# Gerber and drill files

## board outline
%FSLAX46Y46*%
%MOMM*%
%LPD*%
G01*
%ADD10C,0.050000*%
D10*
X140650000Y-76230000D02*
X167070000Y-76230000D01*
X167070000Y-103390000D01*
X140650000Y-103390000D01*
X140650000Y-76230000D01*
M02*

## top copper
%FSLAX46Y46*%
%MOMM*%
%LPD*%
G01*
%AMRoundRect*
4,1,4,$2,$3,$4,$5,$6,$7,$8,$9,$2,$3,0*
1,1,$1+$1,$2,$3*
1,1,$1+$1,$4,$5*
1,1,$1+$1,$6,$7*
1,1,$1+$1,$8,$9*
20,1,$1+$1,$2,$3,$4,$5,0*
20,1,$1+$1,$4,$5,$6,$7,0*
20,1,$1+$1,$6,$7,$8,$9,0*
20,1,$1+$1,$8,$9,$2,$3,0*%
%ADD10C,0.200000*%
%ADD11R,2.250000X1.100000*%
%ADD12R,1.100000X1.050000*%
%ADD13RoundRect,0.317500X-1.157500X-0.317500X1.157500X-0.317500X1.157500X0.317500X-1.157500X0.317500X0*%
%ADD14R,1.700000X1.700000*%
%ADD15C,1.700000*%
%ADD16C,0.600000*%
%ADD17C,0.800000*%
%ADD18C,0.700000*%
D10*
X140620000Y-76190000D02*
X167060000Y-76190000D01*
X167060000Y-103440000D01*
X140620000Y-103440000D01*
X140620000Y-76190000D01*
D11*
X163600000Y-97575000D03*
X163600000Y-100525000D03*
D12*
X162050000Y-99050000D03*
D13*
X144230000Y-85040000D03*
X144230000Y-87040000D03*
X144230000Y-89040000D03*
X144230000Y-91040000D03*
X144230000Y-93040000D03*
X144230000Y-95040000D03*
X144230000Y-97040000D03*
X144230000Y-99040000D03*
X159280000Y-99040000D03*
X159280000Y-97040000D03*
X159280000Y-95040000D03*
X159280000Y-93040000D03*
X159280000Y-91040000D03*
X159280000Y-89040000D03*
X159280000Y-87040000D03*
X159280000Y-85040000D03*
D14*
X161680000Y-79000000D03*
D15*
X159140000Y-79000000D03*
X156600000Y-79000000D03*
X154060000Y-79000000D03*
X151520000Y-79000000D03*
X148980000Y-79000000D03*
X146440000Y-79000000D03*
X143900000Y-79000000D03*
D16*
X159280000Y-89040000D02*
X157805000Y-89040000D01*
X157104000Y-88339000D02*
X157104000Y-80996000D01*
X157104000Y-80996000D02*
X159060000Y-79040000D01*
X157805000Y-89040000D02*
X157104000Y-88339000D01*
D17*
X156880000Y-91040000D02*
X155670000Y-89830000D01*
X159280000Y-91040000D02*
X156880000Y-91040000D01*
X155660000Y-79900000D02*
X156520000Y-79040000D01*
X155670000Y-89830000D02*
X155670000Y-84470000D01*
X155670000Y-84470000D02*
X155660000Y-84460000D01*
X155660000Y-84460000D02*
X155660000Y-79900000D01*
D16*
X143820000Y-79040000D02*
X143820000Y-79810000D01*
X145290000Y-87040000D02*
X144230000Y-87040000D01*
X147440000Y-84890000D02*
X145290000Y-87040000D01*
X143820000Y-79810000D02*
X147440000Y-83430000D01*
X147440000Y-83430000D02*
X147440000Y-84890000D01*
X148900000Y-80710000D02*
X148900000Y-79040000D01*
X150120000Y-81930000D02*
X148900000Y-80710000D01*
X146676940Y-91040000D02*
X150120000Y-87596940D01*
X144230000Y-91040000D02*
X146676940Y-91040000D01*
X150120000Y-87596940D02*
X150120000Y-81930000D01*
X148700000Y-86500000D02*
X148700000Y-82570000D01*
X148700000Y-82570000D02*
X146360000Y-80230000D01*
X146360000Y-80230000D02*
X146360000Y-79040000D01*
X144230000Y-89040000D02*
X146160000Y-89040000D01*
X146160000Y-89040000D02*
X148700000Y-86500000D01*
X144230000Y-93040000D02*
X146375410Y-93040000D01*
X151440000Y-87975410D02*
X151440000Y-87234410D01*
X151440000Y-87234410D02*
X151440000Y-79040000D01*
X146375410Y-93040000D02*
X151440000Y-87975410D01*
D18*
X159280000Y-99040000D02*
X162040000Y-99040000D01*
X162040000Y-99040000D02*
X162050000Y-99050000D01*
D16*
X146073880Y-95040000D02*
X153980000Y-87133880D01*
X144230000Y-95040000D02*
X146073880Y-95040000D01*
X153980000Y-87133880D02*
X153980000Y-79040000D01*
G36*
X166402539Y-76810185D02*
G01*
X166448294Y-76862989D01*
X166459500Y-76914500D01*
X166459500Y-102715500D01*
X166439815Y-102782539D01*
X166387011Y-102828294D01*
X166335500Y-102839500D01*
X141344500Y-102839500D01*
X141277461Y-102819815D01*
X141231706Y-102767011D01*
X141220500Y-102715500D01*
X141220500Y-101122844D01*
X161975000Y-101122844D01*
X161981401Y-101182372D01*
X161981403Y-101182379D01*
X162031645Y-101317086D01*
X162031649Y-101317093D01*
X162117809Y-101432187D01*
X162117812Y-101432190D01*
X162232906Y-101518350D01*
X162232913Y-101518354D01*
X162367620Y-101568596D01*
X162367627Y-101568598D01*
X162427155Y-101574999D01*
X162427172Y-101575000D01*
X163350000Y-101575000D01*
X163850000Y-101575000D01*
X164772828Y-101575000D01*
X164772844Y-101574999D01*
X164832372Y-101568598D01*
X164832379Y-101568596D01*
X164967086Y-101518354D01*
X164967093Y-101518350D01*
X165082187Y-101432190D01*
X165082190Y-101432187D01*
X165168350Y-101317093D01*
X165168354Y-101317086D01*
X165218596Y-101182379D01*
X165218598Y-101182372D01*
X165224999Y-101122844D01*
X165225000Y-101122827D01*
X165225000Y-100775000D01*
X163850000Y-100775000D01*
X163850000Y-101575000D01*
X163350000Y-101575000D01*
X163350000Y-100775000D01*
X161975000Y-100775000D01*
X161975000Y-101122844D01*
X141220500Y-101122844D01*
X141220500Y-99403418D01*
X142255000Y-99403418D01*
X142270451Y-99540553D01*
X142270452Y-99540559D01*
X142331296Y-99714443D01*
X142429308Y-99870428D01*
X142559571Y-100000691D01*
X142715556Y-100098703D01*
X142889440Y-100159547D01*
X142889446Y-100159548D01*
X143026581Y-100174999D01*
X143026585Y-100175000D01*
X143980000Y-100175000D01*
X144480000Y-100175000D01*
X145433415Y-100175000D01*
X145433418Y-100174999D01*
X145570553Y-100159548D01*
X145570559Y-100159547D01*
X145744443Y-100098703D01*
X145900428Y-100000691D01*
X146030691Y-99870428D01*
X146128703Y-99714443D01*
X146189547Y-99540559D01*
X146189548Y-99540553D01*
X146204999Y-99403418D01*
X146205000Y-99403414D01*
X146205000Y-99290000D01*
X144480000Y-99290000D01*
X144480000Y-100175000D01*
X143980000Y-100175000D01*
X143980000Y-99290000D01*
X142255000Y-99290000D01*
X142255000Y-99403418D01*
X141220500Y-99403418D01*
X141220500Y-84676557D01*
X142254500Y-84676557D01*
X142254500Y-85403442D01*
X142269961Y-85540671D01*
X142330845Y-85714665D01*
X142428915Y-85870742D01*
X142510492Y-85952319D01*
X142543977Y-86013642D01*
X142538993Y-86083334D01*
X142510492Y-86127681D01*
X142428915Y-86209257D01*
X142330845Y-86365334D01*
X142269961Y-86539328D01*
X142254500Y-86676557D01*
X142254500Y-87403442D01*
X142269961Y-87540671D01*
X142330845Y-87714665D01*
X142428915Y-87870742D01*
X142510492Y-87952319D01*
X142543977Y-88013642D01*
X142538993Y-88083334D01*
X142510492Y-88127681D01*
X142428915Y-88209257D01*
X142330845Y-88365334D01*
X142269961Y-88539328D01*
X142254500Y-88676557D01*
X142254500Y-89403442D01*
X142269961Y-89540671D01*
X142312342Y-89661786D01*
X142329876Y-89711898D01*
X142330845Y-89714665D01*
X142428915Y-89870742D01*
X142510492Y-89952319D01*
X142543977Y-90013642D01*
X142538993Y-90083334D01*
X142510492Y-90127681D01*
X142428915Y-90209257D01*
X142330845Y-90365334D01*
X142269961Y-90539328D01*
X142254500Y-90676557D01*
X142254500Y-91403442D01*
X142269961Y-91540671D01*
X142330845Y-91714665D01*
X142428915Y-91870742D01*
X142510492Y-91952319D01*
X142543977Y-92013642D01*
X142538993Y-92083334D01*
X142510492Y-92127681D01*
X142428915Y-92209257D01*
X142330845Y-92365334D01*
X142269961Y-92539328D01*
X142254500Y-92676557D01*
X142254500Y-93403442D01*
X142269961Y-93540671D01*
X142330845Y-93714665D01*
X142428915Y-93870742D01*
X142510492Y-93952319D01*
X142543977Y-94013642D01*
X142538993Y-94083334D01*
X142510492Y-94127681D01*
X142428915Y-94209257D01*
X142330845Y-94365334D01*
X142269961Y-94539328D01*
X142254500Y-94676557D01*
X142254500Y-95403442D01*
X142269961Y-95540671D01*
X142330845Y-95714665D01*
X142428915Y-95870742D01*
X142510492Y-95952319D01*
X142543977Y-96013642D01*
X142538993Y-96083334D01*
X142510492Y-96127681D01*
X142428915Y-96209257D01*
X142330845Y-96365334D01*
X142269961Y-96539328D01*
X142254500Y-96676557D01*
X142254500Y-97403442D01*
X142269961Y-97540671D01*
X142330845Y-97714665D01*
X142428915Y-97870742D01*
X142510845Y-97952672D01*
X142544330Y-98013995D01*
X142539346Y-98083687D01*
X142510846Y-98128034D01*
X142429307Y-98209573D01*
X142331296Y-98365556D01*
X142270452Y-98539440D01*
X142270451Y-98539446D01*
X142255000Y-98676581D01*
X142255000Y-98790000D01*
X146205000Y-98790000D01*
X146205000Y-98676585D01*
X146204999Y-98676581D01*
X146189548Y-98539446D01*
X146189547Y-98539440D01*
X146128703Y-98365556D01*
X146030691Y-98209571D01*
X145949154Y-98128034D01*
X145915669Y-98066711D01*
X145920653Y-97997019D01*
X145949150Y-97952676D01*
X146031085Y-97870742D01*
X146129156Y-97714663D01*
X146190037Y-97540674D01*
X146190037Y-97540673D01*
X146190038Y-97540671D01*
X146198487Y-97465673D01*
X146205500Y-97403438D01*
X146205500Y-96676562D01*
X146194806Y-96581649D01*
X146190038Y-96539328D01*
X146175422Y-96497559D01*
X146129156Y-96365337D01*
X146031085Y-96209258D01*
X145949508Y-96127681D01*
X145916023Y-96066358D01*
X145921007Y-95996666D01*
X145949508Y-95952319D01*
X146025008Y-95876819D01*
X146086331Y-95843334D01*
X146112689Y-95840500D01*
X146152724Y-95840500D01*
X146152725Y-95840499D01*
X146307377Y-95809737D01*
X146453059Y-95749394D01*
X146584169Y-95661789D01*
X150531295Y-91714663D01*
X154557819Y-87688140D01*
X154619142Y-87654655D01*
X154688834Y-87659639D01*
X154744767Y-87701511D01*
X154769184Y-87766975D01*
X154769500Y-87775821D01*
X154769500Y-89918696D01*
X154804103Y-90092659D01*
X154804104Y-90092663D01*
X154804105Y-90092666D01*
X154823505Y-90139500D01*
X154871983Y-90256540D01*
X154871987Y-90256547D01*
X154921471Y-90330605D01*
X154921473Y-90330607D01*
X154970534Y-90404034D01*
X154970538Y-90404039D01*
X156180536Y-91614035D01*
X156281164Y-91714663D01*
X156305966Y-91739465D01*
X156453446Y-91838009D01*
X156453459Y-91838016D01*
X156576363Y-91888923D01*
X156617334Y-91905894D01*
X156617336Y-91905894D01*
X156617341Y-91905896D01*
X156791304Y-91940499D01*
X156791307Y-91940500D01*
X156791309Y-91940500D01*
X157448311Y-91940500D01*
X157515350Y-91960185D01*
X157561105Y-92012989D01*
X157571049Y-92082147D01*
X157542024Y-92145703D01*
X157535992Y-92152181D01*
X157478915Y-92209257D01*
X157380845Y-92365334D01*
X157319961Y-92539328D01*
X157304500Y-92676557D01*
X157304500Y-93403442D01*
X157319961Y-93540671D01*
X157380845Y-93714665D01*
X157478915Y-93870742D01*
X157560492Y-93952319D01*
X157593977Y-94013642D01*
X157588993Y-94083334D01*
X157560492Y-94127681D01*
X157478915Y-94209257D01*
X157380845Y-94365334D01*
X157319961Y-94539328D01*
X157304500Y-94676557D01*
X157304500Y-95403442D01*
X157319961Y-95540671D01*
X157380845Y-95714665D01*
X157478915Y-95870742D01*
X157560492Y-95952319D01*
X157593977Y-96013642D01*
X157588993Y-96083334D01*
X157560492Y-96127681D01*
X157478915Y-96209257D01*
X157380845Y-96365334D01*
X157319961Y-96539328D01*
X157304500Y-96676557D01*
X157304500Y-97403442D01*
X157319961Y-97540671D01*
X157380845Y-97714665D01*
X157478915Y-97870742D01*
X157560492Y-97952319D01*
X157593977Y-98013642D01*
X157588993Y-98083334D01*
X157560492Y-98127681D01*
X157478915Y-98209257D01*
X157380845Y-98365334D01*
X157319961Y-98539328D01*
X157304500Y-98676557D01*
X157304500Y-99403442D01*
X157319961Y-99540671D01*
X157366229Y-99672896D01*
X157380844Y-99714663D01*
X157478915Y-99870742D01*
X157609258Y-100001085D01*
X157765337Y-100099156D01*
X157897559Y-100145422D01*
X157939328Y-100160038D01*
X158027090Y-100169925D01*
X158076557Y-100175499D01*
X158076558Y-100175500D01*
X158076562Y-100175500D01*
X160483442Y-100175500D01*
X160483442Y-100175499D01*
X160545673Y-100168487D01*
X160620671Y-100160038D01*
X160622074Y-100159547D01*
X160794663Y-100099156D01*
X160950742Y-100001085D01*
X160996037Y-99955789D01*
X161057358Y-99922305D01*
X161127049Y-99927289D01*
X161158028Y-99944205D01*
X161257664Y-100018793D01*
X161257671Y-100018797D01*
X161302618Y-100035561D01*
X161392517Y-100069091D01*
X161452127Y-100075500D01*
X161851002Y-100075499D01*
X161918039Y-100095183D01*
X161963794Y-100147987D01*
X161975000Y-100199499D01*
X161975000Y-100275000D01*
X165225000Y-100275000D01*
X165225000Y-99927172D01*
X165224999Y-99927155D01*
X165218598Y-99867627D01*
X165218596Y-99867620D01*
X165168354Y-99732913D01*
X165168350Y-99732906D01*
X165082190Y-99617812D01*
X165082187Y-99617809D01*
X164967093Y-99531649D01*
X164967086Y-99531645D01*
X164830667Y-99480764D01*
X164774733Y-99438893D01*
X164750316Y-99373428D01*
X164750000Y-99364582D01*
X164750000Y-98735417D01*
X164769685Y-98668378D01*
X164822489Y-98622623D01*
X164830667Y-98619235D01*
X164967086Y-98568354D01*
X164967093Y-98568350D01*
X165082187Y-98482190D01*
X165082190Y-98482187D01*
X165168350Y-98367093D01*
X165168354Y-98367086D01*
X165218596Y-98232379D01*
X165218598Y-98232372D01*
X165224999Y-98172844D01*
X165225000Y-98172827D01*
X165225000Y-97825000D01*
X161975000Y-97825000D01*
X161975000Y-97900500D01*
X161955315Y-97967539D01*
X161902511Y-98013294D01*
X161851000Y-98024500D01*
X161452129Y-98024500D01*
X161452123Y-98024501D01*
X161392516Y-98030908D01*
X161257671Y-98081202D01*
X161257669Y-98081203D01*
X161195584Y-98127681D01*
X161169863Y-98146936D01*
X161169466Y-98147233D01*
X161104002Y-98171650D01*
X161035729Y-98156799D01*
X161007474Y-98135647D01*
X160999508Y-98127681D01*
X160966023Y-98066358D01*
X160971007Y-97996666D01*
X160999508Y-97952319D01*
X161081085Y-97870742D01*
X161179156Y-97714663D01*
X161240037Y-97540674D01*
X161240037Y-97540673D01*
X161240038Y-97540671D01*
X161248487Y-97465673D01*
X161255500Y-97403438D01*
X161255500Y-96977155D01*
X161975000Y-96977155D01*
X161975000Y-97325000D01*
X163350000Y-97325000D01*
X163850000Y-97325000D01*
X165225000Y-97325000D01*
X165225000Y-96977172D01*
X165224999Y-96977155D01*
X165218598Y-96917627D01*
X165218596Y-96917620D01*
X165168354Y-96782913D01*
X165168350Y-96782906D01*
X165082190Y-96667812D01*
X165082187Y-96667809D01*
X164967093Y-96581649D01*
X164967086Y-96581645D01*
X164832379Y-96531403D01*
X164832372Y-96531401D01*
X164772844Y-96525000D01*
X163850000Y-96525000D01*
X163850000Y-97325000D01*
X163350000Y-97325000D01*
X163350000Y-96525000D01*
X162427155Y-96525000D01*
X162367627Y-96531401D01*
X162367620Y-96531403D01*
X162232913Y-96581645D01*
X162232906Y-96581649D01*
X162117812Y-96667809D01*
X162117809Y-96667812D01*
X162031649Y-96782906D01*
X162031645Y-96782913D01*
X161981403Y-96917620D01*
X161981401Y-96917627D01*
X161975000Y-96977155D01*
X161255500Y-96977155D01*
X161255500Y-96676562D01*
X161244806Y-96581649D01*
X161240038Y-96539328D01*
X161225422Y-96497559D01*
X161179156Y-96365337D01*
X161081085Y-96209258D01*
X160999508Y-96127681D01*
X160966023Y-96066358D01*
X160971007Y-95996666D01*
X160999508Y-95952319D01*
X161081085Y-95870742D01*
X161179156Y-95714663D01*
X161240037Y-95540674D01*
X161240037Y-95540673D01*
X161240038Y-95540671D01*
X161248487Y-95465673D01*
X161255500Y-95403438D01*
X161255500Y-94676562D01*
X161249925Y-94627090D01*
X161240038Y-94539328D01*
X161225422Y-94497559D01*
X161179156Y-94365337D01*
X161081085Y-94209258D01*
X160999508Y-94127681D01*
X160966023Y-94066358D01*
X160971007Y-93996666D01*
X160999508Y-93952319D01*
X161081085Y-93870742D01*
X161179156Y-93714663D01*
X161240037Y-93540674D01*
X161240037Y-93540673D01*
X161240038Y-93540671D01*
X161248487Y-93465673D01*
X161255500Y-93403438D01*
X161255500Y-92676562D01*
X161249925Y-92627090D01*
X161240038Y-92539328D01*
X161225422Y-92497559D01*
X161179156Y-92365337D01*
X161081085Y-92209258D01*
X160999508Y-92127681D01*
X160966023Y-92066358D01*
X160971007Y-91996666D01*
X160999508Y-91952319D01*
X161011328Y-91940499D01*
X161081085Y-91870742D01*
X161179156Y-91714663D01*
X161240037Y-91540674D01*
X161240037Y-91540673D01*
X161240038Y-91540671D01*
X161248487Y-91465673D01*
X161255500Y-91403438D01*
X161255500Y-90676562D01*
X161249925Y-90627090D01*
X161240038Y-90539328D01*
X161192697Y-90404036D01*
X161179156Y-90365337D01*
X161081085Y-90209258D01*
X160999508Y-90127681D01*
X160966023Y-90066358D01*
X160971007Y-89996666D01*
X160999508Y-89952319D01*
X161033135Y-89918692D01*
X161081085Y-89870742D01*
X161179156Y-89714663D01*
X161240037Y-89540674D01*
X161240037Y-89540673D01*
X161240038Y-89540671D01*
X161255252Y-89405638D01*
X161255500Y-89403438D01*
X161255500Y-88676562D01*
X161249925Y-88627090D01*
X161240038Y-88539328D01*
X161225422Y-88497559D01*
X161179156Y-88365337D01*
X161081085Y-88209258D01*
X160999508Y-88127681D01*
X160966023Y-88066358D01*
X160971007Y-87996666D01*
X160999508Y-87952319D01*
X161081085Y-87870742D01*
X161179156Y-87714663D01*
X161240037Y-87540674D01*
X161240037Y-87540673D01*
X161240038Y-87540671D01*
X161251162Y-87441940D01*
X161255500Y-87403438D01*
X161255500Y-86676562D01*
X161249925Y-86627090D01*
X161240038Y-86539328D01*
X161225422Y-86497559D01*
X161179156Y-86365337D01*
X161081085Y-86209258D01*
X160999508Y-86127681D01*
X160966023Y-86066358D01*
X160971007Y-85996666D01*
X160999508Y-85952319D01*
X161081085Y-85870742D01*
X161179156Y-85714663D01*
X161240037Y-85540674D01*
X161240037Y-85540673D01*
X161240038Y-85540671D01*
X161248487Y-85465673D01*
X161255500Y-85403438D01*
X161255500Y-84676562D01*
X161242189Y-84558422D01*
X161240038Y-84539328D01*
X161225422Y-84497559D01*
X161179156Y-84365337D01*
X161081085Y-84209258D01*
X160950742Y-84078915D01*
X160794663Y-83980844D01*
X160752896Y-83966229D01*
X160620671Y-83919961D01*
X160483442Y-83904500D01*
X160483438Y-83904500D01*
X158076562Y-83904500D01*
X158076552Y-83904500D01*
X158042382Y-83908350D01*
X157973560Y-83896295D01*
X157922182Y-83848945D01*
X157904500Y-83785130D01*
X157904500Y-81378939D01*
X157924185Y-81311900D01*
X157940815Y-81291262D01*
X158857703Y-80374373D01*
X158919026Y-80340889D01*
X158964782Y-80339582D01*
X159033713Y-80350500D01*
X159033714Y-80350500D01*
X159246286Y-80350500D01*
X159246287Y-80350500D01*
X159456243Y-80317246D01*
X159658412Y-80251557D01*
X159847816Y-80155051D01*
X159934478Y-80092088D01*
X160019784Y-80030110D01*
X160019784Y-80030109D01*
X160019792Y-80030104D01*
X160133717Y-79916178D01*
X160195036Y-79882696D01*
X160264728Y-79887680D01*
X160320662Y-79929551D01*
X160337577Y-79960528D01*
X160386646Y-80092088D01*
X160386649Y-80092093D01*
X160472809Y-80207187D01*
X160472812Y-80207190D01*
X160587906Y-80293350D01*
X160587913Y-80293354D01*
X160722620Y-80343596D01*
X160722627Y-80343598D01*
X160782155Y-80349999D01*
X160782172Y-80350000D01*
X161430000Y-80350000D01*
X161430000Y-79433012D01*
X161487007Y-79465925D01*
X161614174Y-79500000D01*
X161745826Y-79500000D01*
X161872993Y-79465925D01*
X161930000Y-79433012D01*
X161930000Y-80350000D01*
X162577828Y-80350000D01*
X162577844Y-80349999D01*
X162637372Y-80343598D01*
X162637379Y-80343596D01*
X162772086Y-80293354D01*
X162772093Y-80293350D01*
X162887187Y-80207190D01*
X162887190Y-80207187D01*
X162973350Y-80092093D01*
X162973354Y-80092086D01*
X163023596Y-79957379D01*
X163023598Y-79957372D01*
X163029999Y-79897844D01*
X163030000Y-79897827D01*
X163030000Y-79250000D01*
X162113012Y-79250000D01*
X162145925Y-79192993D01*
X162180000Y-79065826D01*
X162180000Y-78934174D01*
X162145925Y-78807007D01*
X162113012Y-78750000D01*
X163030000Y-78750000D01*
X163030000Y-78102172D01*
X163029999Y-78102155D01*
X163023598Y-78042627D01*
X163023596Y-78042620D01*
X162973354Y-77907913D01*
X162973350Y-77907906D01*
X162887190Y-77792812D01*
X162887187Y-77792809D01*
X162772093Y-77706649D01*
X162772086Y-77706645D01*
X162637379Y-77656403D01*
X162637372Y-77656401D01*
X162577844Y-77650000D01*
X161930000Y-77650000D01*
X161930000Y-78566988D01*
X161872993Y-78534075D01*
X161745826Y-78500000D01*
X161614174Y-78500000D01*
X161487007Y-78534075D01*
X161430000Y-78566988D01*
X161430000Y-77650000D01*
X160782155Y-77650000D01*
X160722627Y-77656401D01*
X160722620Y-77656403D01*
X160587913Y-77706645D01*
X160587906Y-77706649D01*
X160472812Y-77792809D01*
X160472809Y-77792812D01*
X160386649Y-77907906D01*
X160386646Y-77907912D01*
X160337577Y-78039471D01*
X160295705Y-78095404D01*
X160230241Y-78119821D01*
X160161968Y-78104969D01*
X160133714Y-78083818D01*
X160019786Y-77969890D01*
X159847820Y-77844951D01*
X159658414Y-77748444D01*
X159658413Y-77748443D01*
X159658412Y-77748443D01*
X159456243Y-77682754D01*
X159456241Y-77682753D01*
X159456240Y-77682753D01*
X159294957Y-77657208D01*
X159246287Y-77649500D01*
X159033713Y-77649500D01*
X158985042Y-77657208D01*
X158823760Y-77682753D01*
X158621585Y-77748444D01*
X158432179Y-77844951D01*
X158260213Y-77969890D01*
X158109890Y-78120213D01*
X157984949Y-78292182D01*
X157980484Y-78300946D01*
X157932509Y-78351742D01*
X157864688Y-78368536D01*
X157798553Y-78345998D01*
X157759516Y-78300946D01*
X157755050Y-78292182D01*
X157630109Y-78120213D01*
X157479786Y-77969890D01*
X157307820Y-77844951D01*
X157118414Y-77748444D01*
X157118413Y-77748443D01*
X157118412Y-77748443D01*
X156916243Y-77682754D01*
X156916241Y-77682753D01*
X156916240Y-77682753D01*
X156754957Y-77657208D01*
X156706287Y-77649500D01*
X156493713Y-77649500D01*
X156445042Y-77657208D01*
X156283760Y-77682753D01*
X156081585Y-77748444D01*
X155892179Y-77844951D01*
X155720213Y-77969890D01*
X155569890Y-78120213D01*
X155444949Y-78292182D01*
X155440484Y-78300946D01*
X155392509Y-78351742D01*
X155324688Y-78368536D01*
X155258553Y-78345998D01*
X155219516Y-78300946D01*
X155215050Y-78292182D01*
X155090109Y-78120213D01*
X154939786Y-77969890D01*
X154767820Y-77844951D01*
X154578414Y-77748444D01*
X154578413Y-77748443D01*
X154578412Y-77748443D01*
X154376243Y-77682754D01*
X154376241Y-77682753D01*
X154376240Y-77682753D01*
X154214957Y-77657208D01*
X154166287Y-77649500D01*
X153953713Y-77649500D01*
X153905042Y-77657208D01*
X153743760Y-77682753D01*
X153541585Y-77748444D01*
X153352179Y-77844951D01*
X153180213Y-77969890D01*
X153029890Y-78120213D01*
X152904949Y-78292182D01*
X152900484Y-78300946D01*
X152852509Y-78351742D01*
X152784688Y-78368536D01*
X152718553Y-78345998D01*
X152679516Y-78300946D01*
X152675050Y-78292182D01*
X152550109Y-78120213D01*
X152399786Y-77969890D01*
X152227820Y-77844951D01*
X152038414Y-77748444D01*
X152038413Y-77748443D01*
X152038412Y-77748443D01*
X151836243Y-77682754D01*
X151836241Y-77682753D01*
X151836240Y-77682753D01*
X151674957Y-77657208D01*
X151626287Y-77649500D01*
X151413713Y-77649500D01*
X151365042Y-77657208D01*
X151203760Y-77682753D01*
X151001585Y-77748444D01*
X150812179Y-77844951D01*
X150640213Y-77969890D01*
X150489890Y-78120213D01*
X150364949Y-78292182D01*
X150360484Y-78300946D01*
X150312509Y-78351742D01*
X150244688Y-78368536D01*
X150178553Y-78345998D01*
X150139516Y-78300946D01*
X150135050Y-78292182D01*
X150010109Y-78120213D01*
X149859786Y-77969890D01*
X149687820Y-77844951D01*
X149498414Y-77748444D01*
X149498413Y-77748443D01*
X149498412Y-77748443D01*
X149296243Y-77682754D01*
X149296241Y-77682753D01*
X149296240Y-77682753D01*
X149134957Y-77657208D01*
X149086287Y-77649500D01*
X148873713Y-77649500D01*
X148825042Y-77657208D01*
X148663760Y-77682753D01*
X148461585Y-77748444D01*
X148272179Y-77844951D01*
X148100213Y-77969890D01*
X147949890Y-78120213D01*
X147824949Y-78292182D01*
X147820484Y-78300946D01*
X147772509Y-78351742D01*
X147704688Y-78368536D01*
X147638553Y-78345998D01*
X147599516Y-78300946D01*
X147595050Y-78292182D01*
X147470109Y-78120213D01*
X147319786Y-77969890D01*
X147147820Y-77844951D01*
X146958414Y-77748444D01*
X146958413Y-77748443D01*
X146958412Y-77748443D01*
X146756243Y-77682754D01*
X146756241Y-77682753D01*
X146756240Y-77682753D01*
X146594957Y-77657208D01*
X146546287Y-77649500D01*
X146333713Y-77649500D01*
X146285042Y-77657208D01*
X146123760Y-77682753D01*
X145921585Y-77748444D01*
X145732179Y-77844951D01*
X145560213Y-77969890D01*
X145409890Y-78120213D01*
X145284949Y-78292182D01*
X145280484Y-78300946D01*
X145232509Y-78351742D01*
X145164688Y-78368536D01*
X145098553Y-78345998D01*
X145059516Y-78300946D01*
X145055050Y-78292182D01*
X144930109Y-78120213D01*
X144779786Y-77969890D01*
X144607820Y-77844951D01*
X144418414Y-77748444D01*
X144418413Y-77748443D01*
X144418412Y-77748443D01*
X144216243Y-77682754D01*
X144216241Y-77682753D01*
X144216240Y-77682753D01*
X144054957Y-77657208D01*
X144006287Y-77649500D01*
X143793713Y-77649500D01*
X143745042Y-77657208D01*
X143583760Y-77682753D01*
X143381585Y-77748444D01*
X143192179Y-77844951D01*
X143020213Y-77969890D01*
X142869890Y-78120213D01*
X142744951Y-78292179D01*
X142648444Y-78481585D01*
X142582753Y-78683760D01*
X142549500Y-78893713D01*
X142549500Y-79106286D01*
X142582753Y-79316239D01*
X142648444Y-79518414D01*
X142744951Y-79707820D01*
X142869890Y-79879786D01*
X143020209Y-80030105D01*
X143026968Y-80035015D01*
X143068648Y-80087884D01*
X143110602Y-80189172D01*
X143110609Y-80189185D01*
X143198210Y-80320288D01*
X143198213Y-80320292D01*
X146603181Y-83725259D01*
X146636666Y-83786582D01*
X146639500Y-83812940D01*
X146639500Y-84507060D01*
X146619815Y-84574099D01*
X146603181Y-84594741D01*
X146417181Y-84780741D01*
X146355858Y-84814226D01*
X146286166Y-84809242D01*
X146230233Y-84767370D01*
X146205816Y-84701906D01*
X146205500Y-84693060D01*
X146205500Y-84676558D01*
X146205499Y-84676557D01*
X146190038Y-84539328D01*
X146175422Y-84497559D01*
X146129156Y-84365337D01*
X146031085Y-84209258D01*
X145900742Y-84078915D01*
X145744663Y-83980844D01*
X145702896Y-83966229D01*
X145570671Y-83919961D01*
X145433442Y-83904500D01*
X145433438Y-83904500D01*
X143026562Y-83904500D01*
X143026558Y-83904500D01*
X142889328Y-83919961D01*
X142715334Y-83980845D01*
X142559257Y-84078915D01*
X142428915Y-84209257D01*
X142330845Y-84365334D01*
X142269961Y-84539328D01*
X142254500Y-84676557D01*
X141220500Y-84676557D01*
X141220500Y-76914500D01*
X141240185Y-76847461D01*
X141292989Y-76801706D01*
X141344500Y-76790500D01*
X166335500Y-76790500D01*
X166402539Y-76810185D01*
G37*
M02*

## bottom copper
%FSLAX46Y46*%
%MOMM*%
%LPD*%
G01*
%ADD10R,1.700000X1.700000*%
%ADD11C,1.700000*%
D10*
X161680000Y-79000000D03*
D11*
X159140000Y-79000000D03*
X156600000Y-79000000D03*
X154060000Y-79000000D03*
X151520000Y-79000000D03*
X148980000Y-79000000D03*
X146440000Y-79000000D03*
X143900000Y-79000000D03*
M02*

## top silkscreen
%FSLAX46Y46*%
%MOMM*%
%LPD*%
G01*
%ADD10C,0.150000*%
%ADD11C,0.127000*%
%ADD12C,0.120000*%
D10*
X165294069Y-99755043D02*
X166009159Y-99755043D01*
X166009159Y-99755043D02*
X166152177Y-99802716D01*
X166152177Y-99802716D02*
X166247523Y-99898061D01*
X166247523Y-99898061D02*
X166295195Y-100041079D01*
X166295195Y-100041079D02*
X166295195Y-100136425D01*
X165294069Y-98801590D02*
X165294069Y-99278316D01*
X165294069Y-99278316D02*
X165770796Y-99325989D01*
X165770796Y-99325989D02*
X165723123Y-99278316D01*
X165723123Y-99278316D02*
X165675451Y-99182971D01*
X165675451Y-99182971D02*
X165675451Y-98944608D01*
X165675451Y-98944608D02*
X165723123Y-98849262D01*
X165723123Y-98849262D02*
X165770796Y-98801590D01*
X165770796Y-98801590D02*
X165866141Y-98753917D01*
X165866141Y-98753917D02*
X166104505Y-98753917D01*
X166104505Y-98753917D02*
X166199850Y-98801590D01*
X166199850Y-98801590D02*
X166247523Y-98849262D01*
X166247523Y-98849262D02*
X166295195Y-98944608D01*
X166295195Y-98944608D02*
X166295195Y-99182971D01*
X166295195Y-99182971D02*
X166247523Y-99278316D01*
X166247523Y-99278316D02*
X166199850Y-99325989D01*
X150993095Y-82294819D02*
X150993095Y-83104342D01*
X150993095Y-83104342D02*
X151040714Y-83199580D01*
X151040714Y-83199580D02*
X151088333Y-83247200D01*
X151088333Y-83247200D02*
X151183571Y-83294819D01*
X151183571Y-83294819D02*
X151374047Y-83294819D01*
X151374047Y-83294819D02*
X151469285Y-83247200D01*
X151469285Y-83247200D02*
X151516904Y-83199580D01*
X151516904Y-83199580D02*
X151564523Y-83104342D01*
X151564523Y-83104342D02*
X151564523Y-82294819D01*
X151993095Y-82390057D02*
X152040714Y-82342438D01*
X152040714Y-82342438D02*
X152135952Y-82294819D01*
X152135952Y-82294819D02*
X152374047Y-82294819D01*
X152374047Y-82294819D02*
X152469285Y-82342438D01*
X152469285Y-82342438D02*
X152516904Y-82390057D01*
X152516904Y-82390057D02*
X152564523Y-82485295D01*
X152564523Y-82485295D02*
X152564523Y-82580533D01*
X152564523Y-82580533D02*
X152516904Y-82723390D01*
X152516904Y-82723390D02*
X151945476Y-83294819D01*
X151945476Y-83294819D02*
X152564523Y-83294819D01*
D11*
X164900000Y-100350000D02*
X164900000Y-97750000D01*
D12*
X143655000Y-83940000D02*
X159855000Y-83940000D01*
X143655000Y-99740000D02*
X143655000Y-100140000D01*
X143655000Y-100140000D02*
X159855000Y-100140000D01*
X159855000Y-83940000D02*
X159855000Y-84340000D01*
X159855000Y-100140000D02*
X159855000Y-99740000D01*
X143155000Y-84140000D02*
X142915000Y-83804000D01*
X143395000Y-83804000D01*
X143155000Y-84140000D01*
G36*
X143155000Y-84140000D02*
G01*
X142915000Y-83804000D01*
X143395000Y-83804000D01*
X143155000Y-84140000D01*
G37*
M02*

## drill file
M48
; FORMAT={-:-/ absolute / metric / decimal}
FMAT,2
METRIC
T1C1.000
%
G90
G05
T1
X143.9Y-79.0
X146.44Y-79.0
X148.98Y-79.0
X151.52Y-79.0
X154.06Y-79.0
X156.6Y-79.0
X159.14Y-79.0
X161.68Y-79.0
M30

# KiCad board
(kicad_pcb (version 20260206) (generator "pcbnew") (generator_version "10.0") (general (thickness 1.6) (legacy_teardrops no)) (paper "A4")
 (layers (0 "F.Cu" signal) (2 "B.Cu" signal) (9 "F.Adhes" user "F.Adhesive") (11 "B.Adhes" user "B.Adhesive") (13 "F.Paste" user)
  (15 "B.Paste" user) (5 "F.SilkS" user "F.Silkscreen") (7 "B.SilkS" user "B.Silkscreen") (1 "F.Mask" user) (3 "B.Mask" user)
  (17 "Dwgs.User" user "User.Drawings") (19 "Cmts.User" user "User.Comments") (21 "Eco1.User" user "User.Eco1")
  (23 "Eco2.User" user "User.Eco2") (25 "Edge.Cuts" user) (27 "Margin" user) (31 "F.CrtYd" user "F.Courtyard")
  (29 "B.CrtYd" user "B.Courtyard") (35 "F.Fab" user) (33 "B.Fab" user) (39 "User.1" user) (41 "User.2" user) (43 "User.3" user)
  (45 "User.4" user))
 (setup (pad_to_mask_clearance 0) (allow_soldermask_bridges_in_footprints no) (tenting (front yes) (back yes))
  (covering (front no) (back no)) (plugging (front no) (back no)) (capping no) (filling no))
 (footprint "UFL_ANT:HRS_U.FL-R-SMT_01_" (layer "F.Cu") (at 163.6 99.05 -90)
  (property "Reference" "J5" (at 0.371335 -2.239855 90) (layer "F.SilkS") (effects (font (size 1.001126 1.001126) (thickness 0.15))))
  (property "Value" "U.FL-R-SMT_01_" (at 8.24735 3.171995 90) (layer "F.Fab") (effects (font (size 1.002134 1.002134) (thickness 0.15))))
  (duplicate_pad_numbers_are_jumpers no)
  (fp_line (start 1.3 -1.3) (end -1.3 -1.3) (stroke (width 0.127) (type solid)) (layer "F.SilkS"))
  (pad "1" smd rect (at -1.475 0 270) (size 1.1 2.25) (layers "F.Cu" "F.Mask" "F.Paste") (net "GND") (solder_mask_margin 0.102))
  (pad "2" smd rect (at 1.475 0 270) (size 1.1 2.25) (layers "F.Cu" "F.Mask" "F.Paste") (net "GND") (solder_mask_margin 0.102))
  (pad "3" smd rect (at 0 1.55 270) (size 1.05 1.1) (layers "F.Cu" "F.Mask" "F.Paste") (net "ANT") (solder_mask_margin 0.102))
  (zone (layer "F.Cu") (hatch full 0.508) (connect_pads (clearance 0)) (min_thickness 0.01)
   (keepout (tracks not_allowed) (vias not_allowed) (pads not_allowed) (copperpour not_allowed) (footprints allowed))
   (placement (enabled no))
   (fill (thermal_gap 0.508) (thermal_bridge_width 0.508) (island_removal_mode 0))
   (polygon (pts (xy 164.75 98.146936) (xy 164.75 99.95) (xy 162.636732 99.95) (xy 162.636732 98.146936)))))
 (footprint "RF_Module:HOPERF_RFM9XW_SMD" (layer "F.Cu") (at 151.755 92.04)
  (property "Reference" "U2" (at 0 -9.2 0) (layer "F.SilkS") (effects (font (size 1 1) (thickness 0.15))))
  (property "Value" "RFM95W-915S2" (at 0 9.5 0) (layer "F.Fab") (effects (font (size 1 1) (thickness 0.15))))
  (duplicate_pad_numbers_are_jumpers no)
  (fp_line (start -8.1 -8.1) (end 8.1 -8.1) (stroke (width 0.12) (type solid)) (layer "F.SilkS"))
  (fp_line (start -8.1 7.7) (end -8.1 8.1) (stroke (width 0.12) (type solid)) (layer "F.SilkS"))
  (fp_line (start -8.1 8.1) (end 8.1 8.1) (stroke (width 0.12) (type solid)) (layer "F.SilkS"))
  (fp_line (start 8.1 -8.1) (end 8.1 -7.7) (stroke (width 0.12) (type solid)) (layer "F.SilkS"))
  (fp_line (start 8.1 8.1) (end 8.1 7.7) (stroke (width 0.12) (type solid)) (layer "F.SilkS"))
  (fp_poly
   (pts (xy -8.6 -7.9) (xy -8.84 -8.236) (xy -8.36 -8.236) (xy -8.6 -7.9)) (stroke (width 0.12) (type solid)) (fill yes) (layer "F.SilkS"))
  (pad "1" smd roundrect (at -7.525 -7) (size 2.95 1.27) (layers "F.Cu" "F.Mask" "F.Paste") (roundrect_rratio 0.25)
   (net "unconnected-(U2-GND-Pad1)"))
  (pad "2" smd roundrect (at -7.525 -5) (size 2.95 1.27) (layers "F.Cu" "F.Mask" "F.Paste") (roundrect_rratio 0.25) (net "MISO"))
  (pad "3" smd roundrect (at -7.525 -3) (size 2.95 1.27) (layers "F.Cu" "F.Mask" "F.Paste") (roundrect_rratio 0.25) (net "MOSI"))
  (pad "4" smd roundrect (at -7.525 -1) (size 2.95 1.27) (layers "F.Cu" "F.Mask" "F.Paste") (roundrect_rratio 0.25) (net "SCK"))
  (pad "5" smd roundrect (at -7.525 1) (size 2.95 1.27) (layers "F.Cu" "F.Mask" "F.Paste") (roundrect_rratio 0.25) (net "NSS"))
  (pad "6" smd roundrect (at -7.525 3) (size 2.95 1.27) (layers "F.Cu" "F.Mask" "F.Paste") (roundrect_rratio 0.25) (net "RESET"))
  (pad "7" smd roundrect (at -7.525 5) (size 2.95 1.27) (layers "F.Cu" "F.Mask" "F.Paste") (roundrect_rratio 0.25)
   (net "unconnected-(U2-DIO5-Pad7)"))
  (pad "8" smd roundrect (at -7.525 7) (size 2.95 1.27) (layers "F.Cu" "F.Mask" "F.Paste") (roundrect_rratio 0.25) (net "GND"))
  (pad "9" smd roundrect (at 7.525 7) (size 2.95 1.27) (layers "F.Cu" "F.Mask" "F.Paste") (roundrect_rratio 0.25) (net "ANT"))
  (pad "10" smd roundrect (at 7.525 5) (size 2.95 1.27) (layers "F.Cu" "F.Mask" "F.Paste") (roundrect_rratio 0.25)
   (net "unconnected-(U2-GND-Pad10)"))
  (pad "11" smd roundrect (at 7.525 3) (size 2.95 1.27) (layers "F.Cu" "F.Mask" "F.Paste") (roundrect_rratio 0.25)
   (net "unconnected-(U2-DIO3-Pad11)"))
  (pad "12" smd roundrect (at 7.525 1) (size 2.95 1.27) (layers "F.Cu" "F.Mask" "F.Paste") (roundrect_rratio 0.25)
   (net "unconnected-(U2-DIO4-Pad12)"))
  (pad "13" smd roundrect (at 7.525 -1) (size 2.95 1.27) (layers "F.Cu" "F.Mask" "F.Paste") (roundrect_rratio 0.25) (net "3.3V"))
  (pad "14" smd roundrect (at 7.525 -3) (size 2.95 1.27) (layers "F.Cu" "F.Mask" "F.Paste") (roundrect_rratio 0.25) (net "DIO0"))
  (pad "15" smd roundrect (at 7.525 -5) (size 2.95 1.27) (layers "F.Cu" "F.Mask" "F.Paste") (roundrect_rratio 0.25)
   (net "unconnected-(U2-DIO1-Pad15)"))
  (pad "16" smd roundrect (at 7.525 -7) (size 2.95 1.27) (layers "F.Cu" "F.Mask" "F.Paste") (roundrect_rratio 0.25)
   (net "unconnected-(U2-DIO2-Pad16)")))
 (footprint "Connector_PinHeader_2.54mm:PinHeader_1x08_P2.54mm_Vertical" (layer "B.Cu") (at 161.68 79 90)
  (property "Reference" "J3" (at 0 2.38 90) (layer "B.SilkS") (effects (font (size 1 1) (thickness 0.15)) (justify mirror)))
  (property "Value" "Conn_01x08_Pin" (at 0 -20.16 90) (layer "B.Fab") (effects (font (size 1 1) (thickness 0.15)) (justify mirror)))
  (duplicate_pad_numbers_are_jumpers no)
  (pad "1" thru_hole rect (at 0 0 90) (size 1.7 1.7) (drill 1) (layers "*.Cu" "*.Mask") (remove_unused_layers no) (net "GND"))
  (pad "2" thru_hole circle (at 0 -2.54 90) (size 1.7 1.7) (drill 1) (layers "*.Cu" "*.Mask") (remove_unused_layers no) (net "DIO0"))
  (pad "3" thru_hole circle (at 0 -5.08 90) (size 1.7 1.7) (drill 1) (layers "*.Cu" "*.Mask") (remove_unused_layers no) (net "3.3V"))
  (pad "4" thru_hole circle (at 0 -7.62 90) (size 1.7 1.7) (drill 1) (layers "*.Cu" "*.Mask") (remove_unused_layers no) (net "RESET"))
  (pad "5" thru_hole circle (at 0 -10.16 90) (size 1.7 1.7) (drill 1) (layers "*.Cu" "*.Mask") (remove_unused_layers no) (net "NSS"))
  (pad "6" thru_hole circle (at 0 -12.7 90) (size 1.7 1.7) (drill 1) (layers "*.Cu" "*.Mask") (remove_unused_layers no) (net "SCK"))
  (pad "7" thru_hole circle (at 0 -15.24 90) (size 1.7 1.7) (drill 1) (layers "*.Cu" "*.Mask") (remove_unused_layers no) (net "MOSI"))
  (pad "8" thru_hole circle (at 0 -17.78 90) (size 1.7 1.7) (drill 1) (layers "*.Cu" "*.Mask") (remove_unused_layers no) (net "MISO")))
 (gr_rect (start 140.62 76.19) (end 167.06 103.44) (stroke (width 0.2) (type default)) (fill no) (layer "F.Cu") (net "DIO0"))
 (gr_rect (start 140.65 76.23) (end 167.07 103.39) (stroke (width 0.05) (type default)) (fill no) (layer "Edge.Cuts"))
 (segment (start 159.28 89.04) (end 157.805 89.04) (width 0.6) (layer "F.Cu") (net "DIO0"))
 (segment (start 157.104 88.339) (end 157.104 80.996) (width 0.6) (layer "F.Cu") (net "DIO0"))
 (segment (start 157.104 80.996) (end 159.06 79.04) (width 0.6) (layer "F.Cu") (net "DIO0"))
 (segment (start 157.805 89.04) (end 157.104 88.339) (width 0.6) (layer "F.Cu") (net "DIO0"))
 (segment (start 156.88 91.04) (end 155.67 89.83) (width 0.8) (layer "F.Cu") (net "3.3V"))
 (segment (start 159.28 91.04) (end 156.88 91.04) (width 0.8) (layer "F.Cu") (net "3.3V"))
 (segment (start 155.66 79.9) (end 156.52 79.04) (width 0.8) (layer "F.Cu") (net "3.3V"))
 (segment (start 155.67 89.83) (end 155.67 84.47) (width 0.8) (layer "F.Cu") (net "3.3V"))
 (segment (start 155.67 84.47) (end 155.66 84.46) (width 0.8) (layer "F.Cu") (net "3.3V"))
 (segment (start 155.66 84.46) (end 155.66 79.9) (width 0.8) (layer "F.Cu") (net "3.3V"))
 (segment (start 143.82 79.04) (end 143.82 79.81) (width 0.6) (layer "F.Cu") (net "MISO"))
 (segment (start 145.29 87.04) (end 144.23 87.04) (width 0.6) (layer "F.Cu") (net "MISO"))
 (segment (start 147.44 84.89) (end 145.29 87.04) (width 0.6) (layer "F.Cu") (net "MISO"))
 (segment (start 143.82 79.81) (end 147.44 83.43) (width 0.6) (layer "F.Cu") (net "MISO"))
 (segment (start 147.44 83.43) (end 147.44 84.89) (width 0.6) (layer "F.Cu") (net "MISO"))
 (segment (start 148.9 80.71) (end 148.9 79.04) (width 0.6) (layer "F.Cu") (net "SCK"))
 (segment (start 150.12 81.93) (end 148.9 80.71) (width 0.6) (layer "F.Cu") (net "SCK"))
 (segment (start 146.67694 91.04) (end 150.12 87.59694) (width 0.6) (layer "F.Cu") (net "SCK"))
 (segment (start 144.23 91.04) (end 146.67694 91.04) (width 0.6) (layer "F.Cu") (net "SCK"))
 (segment (start 150.12 87.59694) (end 150.12 81.93) (width 0.6) (layer "F.Cu") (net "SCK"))
 (segment (start 148.7 86.5) (end 148.7 82.57) (width 0.6) (layer "F.Cu") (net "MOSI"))
 (segment (start 148.7 82.57) (end 146.36 80.23) (width 0.6) (layer "F.Cu") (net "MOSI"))
 (segment (start 146.36 80.23) (end 146.36 79.04) (width 0.6) (layer "F.Cu") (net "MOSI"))
 (segment (start 144.23 89.04) (end 146.16 89.04) (width 0.6) (layer "F.Cu") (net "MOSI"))
 (segment (start 146.16 89.04) (end 148.7 86.5) (width 0.6) (layer "F.Cu") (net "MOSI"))
 (segment (start 144.23 93.04) (end 146.37541 93.04) (width 0.6) (layer "F.Cu") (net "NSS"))
 (segment (start 151.44 87.97541) (end 151.44 87.23441) (width 0.6) (layer "F.Cu") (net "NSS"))
 (segment (start 151.44 87.23441) (end 151.44 79.04) (width 0.6) (layer "F.Cu") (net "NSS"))
 (segment (start 146.37541 93.04) (end 151.44 87.97541) (width 0.6) (layer "F.Cu") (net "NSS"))
 (segment (start 159.28 99.04) (end 162.04 99.04) (width 0.7) (layer "F.Cu") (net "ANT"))
 (segment (start 162.04 99.04) (end 162.05 99.05) (width 0.7) (layer "F.Cu") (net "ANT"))
 (segment (start 146.07388 95.04) (end 153.98 87.13388) (width 0.6) (layer "F.Cu") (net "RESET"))
 (segment (start 144.23 95.04) (end 146.07388 95.04) (width 0.6) (layer "F.Cu") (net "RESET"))
 (segment (start 153.98 87.13388) (end 153.98 79.04) (width 0.6) (layer "F.Cu") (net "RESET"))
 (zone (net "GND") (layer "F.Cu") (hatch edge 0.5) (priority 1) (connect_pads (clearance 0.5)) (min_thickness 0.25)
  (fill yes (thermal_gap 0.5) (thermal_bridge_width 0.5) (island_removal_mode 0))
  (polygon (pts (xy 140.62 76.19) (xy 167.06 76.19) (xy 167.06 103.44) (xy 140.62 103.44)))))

